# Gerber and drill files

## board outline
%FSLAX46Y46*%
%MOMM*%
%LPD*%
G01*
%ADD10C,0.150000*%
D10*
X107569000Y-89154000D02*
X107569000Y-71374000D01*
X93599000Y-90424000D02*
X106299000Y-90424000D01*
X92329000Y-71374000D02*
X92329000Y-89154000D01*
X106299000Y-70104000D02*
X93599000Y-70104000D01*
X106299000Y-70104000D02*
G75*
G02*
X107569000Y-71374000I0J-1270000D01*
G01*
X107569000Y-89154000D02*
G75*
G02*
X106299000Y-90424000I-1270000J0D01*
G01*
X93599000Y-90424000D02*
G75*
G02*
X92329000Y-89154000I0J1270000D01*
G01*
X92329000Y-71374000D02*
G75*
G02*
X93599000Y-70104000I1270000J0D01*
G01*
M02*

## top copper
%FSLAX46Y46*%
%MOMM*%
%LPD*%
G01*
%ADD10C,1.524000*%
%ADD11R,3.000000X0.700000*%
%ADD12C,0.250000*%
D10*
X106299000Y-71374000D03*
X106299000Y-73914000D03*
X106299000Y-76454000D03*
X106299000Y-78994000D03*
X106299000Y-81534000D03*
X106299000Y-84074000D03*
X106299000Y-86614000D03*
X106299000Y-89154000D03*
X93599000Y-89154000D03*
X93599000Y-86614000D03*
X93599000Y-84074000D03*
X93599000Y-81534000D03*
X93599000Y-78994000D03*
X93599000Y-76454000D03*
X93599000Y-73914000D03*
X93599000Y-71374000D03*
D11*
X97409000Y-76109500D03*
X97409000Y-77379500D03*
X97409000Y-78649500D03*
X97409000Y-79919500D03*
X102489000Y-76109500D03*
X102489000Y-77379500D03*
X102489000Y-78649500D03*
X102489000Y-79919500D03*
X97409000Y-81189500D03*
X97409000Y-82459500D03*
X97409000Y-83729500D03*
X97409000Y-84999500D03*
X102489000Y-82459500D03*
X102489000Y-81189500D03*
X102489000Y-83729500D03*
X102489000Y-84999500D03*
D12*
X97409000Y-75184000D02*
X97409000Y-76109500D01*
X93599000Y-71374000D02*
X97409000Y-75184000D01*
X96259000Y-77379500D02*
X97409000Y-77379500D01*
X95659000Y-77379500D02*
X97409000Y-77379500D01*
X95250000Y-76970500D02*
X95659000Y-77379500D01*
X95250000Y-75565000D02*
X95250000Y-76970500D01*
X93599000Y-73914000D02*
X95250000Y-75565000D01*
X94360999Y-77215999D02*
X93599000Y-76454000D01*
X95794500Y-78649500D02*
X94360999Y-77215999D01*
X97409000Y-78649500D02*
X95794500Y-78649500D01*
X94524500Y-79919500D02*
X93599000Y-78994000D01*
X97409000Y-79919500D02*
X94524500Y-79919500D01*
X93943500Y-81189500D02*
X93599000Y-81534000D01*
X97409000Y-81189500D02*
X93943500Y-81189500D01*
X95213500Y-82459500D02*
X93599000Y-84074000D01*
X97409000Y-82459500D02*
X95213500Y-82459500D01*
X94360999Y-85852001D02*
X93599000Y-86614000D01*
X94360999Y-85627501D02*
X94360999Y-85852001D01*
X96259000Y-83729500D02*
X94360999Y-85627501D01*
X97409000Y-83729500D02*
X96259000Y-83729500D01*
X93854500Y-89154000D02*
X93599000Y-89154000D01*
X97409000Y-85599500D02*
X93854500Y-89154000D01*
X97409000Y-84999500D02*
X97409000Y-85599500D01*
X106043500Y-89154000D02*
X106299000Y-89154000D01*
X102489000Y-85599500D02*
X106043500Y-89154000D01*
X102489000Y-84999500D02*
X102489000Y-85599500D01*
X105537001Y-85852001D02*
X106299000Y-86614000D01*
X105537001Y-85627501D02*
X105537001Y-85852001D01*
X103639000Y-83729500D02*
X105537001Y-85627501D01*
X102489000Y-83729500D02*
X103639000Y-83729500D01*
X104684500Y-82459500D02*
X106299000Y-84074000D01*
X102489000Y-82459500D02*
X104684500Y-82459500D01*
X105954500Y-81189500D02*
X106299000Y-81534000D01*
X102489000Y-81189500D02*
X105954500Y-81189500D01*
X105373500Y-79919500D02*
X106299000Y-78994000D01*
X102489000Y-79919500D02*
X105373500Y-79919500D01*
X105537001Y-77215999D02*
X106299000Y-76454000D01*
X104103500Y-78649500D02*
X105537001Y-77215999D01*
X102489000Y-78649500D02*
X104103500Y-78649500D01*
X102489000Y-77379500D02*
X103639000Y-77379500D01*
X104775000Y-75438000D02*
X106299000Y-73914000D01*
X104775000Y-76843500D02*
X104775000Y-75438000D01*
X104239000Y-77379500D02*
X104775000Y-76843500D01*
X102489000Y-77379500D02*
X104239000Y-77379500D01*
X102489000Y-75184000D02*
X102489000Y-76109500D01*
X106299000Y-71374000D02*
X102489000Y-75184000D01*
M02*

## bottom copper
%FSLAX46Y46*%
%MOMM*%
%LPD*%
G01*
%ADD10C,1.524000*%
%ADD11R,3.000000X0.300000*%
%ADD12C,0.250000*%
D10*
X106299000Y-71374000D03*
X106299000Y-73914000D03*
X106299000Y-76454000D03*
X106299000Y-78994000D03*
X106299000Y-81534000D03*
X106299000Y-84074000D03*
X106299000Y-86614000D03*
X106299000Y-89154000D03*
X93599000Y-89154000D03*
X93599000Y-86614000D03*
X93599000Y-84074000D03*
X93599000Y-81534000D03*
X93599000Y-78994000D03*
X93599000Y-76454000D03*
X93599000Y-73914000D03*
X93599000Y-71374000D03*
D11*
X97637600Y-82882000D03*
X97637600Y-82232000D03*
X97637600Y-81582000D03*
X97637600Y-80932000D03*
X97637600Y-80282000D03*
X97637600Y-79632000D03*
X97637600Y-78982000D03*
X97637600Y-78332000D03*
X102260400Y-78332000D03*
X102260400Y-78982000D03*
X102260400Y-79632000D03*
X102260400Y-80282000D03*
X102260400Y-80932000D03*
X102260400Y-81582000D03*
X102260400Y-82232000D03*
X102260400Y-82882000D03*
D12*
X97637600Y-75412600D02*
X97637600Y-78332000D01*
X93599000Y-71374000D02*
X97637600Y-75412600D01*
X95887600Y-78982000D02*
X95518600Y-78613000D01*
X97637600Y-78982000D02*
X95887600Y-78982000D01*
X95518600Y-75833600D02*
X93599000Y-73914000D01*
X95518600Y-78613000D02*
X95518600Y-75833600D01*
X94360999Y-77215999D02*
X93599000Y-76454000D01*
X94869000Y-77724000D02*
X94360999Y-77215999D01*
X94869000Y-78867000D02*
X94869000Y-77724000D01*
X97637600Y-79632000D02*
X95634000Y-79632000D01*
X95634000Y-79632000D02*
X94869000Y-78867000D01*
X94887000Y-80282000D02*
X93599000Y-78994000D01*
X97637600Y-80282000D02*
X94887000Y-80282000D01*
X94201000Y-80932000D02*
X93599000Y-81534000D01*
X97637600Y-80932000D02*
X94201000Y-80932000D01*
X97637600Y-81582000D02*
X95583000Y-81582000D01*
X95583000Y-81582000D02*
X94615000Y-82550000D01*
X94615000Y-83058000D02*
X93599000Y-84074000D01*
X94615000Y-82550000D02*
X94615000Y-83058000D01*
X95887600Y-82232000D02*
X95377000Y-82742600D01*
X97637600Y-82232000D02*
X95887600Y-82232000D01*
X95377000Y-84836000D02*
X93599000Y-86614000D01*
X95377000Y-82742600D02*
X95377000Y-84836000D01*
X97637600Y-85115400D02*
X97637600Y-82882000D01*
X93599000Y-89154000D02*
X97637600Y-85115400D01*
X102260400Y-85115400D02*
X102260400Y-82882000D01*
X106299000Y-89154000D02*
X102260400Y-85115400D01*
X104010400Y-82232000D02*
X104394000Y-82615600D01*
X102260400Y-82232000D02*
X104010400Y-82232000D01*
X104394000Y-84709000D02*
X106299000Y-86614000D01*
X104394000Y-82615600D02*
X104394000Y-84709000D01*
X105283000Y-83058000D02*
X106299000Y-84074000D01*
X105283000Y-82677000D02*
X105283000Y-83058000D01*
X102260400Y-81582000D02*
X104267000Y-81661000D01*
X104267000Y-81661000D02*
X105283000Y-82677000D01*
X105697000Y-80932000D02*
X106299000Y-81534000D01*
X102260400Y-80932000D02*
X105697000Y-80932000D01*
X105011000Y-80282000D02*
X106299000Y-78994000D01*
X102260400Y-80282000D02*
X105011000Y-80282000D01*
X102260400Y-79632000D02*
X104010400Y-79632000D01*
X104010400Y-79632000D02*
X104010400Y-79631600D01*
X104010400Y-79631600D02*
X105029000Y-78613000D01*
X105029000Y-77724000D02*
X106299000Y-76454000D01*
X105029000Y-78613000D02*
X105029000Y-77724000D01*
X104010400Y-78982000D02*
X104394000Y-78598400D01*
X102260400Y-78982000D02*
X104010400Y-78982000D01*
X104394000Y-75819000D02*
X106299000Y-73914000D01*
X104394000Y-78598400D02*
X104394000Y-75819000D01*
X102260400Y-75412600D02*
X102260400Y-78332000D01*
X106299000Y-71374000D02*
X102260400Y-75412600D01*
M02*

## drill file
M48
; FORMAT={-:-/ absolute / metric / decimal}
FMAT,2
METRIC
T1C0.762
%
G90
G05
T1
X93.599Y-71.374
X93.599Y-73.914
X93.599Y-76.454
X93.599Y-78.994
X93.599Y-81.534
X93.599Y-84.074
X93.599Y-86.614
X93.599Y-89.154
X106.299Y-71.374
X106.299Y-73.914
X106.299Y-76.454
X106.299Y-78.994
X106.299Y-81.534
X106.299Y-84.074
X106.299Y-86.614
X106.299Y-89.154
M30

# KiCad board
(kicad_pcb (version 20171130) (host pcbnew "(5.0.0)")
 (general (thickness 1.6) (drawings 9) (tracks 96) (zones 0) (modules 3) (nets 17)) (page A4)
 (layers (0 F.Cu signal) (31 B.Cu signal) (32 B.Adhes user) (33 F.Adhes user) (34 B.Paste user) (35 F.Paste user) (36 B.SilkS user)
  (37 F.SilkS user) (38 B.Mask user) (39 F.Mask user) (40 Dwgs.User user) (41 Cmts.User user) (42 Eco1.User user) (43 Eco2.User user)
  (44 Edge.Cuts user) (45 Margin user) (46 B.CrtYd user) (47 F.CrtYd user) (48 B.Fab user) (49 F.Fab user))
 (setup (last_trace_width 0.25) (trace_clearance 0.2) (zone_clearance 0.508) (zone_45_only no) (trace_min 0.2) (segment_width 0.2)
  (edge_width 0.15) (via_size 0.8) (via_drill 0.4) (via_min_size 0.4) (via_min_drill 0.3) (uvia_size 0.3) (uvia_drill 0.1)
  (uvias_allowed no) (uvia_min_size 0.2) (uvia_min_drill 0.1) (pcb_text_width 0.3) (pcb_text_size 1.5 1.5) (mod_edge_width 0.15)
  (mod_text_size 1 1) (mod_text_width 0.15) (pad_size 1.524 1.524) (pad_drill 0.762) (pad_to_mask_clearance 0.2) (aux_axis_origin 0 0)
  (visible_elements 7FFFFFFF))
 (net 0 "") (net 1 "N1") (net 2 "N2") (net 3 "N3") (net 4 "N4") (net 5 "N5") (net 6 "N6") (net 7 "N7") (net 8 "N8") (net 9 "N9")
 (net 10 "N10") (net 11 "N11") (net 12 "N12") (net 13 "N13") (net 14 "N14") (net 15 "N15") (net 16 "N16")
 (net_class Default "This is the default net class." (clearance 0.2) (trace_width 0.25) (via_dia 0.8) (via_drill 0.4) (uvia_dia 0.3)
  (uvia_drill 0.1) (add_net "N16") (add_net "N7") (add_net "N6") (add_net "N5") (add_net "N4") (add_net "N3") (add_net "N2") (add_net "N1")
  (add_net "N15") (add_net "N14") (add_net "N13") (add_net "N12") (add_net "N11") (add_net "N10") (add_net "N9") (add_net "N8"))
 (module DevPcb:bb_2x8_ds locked (layer F.Cu) (at 93.599 71.374)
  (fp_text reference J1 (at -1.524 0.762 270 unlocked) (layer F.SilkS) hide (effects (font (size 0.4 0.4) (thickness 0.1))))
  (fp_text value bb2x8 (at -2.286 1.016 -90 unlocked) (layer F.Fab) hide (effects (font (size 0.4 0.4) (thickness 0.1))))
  (pad 16 thru_hole circle (at 12.7 0) (size 1.524 1.524) (drill 0.762) (layers *.Cu *.Mask) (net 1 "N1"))
  (pad 15 thru_hole circle (at 12.7 2.54) (size 1.524 1.524) (drill 0.762) (layers *.Cu *.Mask) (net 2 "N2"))
  (pad 14 thru_hole circle (at 12.7 5.08) (size 1.524 1.524) (drill 0.762) (layers *.Cu *.Mask) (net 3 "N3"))
  (pad 13 thru_hole circle (at 12.7 7.62) (size 1.524 1.524) (drill 0.762) (layers *.Cu *.Mask) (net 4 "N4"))
  (pad 12 thru_hole circle (at 12.7 10.16) (size 1.524 1.524) (drill 0.762) (layers *.Cu *.Mask) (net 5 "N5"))
  (pad 11 thru_hole circle (at 12.7 12.7) (size 1.524 1.524) (drill 0.762) (layers *.Cu *.Mask) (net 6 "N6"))
  (pad 10 thru_hole circle (at 12.7 15.24) (size 1.524 1.524) (drill 0.762) (layers *.Cu *.Mask) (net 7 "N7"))
  (pad 9 thru_hole circle (at 12.7 17.78) (size 1.524 1.524) (drill 0.762) (layers *.Cu *.Mask) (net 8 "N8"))
  (pad 8 thru_hole circle (at 0 17.78) (size 1.524 1.524) (drill 0.762) (layers *.Cu *.Mask) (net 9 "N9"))
  (pad 7 thru_hole circle (at 0 15.24) (size 1.524 1.524) (drill 0.762) (layers *.Cu *.Mask) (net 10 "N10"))
  (pad 6 thru_hole circle (at 0 12.7) (size 1.524 1.524) (drill 0.762) (layers *.Cu *.Mask) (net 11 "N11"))
  (pad 5 thru_hole circle (at 0 10.16) (size 1.524 1.524) (drill 0.762) (layers *.Cu *.Mask) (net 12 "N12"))
  (pad 4 thru_hole circle (at 0 7.62) (size 1.524 1.524) (drill 0.762) (layers *.Cu *.Mask) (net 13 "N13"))
  (pad 3 thru_hole circle (at 0 5.08) (size 1.524 1.524) (drill 0.762) (layers *.Cu *.Mask) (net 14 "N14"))
  (pad 2 thru_hole circle (at 0 2.54) (size 1.524 1.524) (drill 0.762) (layers *.Cu *.Mask) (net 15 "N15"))
  (pad 1 thru_hole circle (at 0 0) (size 1.524 1.524) (drill 0.762) (layers *.Cu *.Mask) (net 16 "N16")))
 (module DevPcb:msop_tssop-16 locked (layer B.Cu) (at 99.9744 77.062 180)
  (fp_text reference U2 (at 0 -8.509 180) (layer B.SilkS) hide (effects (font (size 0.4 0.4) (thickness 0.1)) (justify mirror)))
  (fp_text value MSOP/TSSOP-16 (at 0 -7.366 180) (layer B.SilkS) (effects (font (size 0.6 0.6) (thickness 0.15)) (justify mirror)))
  (pad 9 smd rect (at 2.3368 -5.82 180) (size 3 0.3) (layers B.Cu B.Paste B.Mask) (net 9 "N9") (solder_mask_margin 0.1))
  (pad 10 smd rect (at 2.3368 -5.17 180) (size 3 0.3) (layers B.Cu B.Paste B.Mask) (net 10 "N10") (solder_mask_margin 0.1))
  (pad 11 smd rect (at 2.3368 -4.52 180) (size 3 0.3) (layers B.Cu B.Paste B.Mask) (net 11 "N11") (solder_mask_margin 0.1))
  (pad 12 smd rect (at 2.3368 -3.87 180) (size 3 0.3) (layers B.Cu B.Paste B.Mask) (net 12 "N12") (solder_mask_margin 0.1))
  (pad 13 smd rect (at 2.3368 -3.22 180) (size 3 0.3) (layers B.Cu B.Paste B.Mask) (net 13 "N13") (solder_mask_margin 0.1))
  (pad 14 smd rect (at 2.3368 -2.57 180) (size 3 0.3) (layers B.Cu B.Paste B.Mask) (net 14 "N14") (solder_mask_margin 0.1))
  (pad 15 smd rect (at 2.3368 -1.92 180) (size 3 0.3) (layers B.Cu B.Paste B.Mask) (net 15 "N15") (solder_mask_margin 0.1))
  (pad 16 smd rect (at 2.3368 -1.27) (size 3 0.3) (layers B.Cu B.Paste B.Mask) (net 16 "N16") (solder_mask_margin 0.1))
  (pad 1 smd rect (at -2.286 -1.27 180) (size 3 0.3) (layers B.Cu B.Paste B.Mask) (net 1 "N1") (solder_mask_margin 0.1))
  (pad 2 smd rect (at -2.286 -1.92 180) (size 3 0.3) (layers B.Cu B.Paste B.Mask) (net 2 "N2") (solder_mask_margin 0.1))
  (pad 3 smd rect (at -2.286 -2.57 180) (size 3 0.3) (layers B.Cu B.Paste B.Mask) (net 3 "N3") (solder_mask_margin 0.1))
  (pad 4 smd rect (at -2.286 -3.22 180) (size 3 0.3) (layers B.Cu B.Paste B.Mask) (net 4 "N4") (solder_mask_margin 0.1))
  (pad 5 smd rect (at -2.286 -3.87 180) (size 3 0.3) (layers B.Cu B.Paste B.Mask) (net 5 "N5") (solder_mask_margin 0.1))
  (pad 6 smd rect (at -2.286 -4.52 180) (size 3 0.3) (layers B.Cu B.Paste B.Mask) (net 6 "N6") (solder_mask_margin 0.1))
  (pad 7 smd rect (at -2.286 -5.17 180) (size 3 0.3) (layers B.Cu B.Paste B.Mask) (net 7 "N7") (solder_mask_margin 0.1))
  (pad 8 smd rect (at -2.286 -5.82 180) (size 3 0.3) (layers B.Cu B.Paste B.Mask) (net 8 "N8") (solder_mask_margin 0.1)))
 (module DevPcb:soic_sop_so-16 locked (layer F.Cu) (at 99.949 74.8395)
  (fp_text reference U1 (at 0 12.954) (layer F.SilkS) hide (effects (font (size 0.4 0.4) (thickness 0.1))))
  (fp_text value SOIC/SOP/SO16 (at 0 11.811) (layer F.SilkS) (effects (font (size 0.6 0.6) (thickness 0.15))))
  (pad 1 smd rect (at -2.54 1.27 90) (size 0.7 3) (layers F.Cu F.Paste F.Mask) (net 16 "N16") (solder_mask_margin 0.1))
  (pad 2 smd rect (at -2.54 2.54 90) (size 0.7 3) (layers F.Cu F.Paste F.Mask) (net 15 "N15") (solder_mask_margin 0.1))
  (pad 3 smd rect (at -2.54 3.81 90) (size 0.7 3) (layers F.Cu F.Paste F.Mask) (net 14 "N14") (solder_mask_margin 0.1))
  (pad 4 smd rect (at -2.54 5.08 90) (size 0.7 3) (layers F.Cu F.Paste F.Mask) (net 13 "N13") (solder_mask_margin 0.1))
  (pad 16 smd rect (at 2.54 1.27 90) (size 0.7 3) (layers F.Cu F.Paste F.Mask) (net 1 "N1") (solder_mask_margin 0.1))
  (pad 15 smd rect (at 2.54 2.54 90) (size 0.7 3) (layers F.Cu F.Paste F.Mask) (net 2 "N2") (solder_mask_margin 0.1))
  (pad 14 smd rect (at 2.54 3.81 90) (size 0.7 3) (layers F.Cu F.Paste F.Mask) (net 3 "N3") (solder_mask_margin 0.1))
  (pad 13 smd rect (at 2.54 5.08 90) (size 0.7 3) (layers F.Cu F.Paste F.Mask) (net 4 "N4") (solder_mask_margin 0.1))
  (pad 5 smd rect (at -2.54 6.35 90) (size 0.7 3) (layers F.Cu F.Paste F.Mask) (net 12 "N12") (solder_mask_margin 0.1))
  (pad 6 smd rect (at -2.54 7.62 90) (size 0.7 3) (layers F.Cu F.Paste F.Mask) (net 11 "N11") (solder_mask_margin 0.1))
  (pad 7 smd rect (at -2.54 8.89 90) (size 0.7 3) (layers F.Cu F.Paste F.Mask) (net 10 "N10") (solder_mask_margin 0.1))
  (pad 8 smd rect (at -2.54 10.16 90) (size 0.7 3) (layers F.Cu F.Paste F.Mask) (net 9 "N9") (solder_mask_margin 0.1))
  (pad 11 smd rect (at 2.54 7.62 90) (size 0.7 3) (layers F.Cu F.Paste F.Mask) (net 6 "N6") (solder_mask_margin 0.1))
  (pad 12 smd rect (at 2.54 6.35 90) (size 0.7 3) (layers F.Cu F.Paste F.Mask) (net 5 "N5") (solder_mask_margin 0.1))
  (pad 10 smd rect (at 2.54 8.89 90) (size 0.7 3) (layers F.Cu F.Paste F.Mask) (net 7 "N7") (solder_mask_margin 0.1))
  (pad 9 smd rect (at 2.54 10.16 90) (size 0.7 3) (layers F.Cu F.Paste F.Mask) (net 8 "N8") (solder_mask_margin 0.1)))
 (gr_line (start 107.569 89.154) (end 107.569 71.374) (layer Edge.Cuts) (width 0.15))
 (gr_line (start 93.599 90.424) (end 106.299 90.424) (layer Edge.Cuts) (width 0.15))
 (gr_line (start 92.329 71.374) (end 92.329 89.154) (layer Edge.Cuts) (width 0.15))
 (gr_line (start 106.299 70.104) (end 93.599 70.104) (layer Edge.Cuts) (width 0.15))
 (gr_arc (start 106.299 71.374) (end 107.569 71.374) (angle -90) (layer Edge.Cuts) (width 0.15))
 (gr_arc (start 106.299 89.154) (end 106.299 90.424) (angle -90) (layer Edge.Cuts) (width 0.15))
 (gr_arc (start 93.599 89.154) (end 92.329 89.154) (angle -90) (layer Edge.Cuts) (width 0.15))
 (gr_arc (start 93.599 71.374) (end 93.599 70.104) (angle -90) (layer Edge.Cuts) (width 0.15))
 (segment (start 97.409 75.184) (end 97.409 76.1095) (width 0.25) (layer F.Cu) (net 16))
 (segment (start 93.599 71.374) (end 97.409 75.184) (width 0.25) (layer F.Cu) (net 16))
 (segment (start 97.6376 75.4126) (end 97.6376 78.332) (width 0.25) (layer B.Cu) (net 16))
 (segment (start 93.599 71.374) (end 97.6376 75.4126) (width 0.25) (layer B.Cu) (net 16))
 (segment (start 96.259 77.3795) (end 97.409 77.3795) (width 0.25) (layer F.Cu) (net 15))
 (segment (start 95.659 77.3795) (end 97.409 77.3795) (width 0.25) (layer F.Cu) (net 15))
 (segment (start 95.25 76.9705) (end 95.659 77.3795) (width 0.25) (layer F.Cu) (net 15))
 (segment (start 95.25 75.565) (end 95.25 76.9705) (width 0.25) (layer F.Cu) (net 15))
 (segment (start 93.599 73.914) (end 95.25 75.565) (width 0.25) (layer F.Cu) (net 15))
 (segment (start 95.8876 78.982) (end 95.5186 78.613) (width 0.25) (layer B.Cu) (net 15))
 (segment (start 97.6376 78.982) (end 95.8876 78.982) (width 0.25) (layer B.Cu) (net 15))
 (segment (start 95.5186 75.8336) (end 93.599 73.914) (width 0.25) (layer B.Cu) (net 15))
 (segment (start 95.5186 78.613) (end 95.5186 75.8336) (width 0.25) (layer B.Cu) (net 15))
 (segment (start 94.360999 77.215999) (end 93.599 76.454) (width 0.25) (layer F.Cu) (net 14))
 (segment (start 95.7945 78.6495) (end 94.360999 77.215999) (width 0.25) (layer F.Cu) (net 14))
 (segment (start 97.409 78.6495) (end 95.7945 78.6495) (width 0.25) (layer F.Cu) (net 14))
 (segment (start 94.360999 77.215999) (end 93.599 76.454) (width 0.25) (layer B.Cu) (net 14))
 (segment (start 94.869 77.724) (end 94.360999 77.215999) (width 0.25) (layer B.Cu) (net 14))
 (segment (start 94.869 78.867) (end 94.869 77.724) (width 0.25) (layer B.Cu) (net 14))
 (segment (start 97.6376 79.632) (end 95.634 79.632) (width 0.25) (layer B.Cu) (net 14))
 (segment (start 95.634 79.632) (end 94.869 78.867) (width 0.25) (layer B.Cu) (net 14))
 (segment (start 94.5245 79.9195) (end 93.599 78.994) (width 0.25) (layer F.Cu) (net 13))
 (segment (start 97.409 79.9195) (end 94.5245 79.9195) (width 0.25) (layer F.Cu) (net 13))
 (segment (start 94.887 80.282) (end 93.599 78.994) (width 0.25) (layer B.Cu) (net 13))
 (segment (start 97.6376 80.282) (end 94.887 80.282) (width 0.25) (layer B.Cu) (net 13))
 (segment (start 93.9435 81.1895) (end 93.599 81.534) (width 0.25) (layer F.Cu) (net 12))
 (segment (start 97.409 81.1895) (end 93.9435 81.1895) (width 0.25) (layer F.Cu) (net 12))
 (segment (start 94.201 80.932) (end 93.599 81.534) (width 0.25) (layer B.Cu) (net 12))
 (segment (start 97.6376 80.932) (end 94.201 80.932) (width 0.25) (layer B.Cu) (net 12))
 (segment (start 95.2135 82.4595) (end 93.599 84.074) (width 0.25) (layer F.Cu) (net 11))
 (segment (start 97.409 82.4595) (end 95.2135 82.4595) (width 0.25) (layer F.Cu) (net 11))
 (segment (start 97.6376 81.582) (end 95.583 81.582) (width 0.25) (layer B.Cu) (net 11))
 (segment (start 95.583 81.582) (end 94.615 82.55) (width 0.25) (layer B.Cu) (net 11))
 (segment (start 94.615 83.058) (end 93.599 84.074) (width 0.25) (layer B.Cu) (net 11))
 (segment (start 94.615 82.55) (end 94.615 83.058) (width 0.25) (layer B.Cu) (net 11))
 (segment (start 94.360999 85.852001) (end 93.599 86.614) (width 0.25) (layer F.Cu) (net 10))
 (segment (start 94.360999 85.627501) (end 94.360999 85.852001) (width 0.25) (layer F.Cu) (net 10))
 (segment (start 96.259 83.7295) (end 94.360999 85.627501) (width 0.25) (layer F.Cu) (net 10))
 (segment (start 97.409 83.7295) (end 96.259 83.7295) (width 0.25) (layer F.Cu) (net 10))
 (segment (start 95.8876 82.232) (end 95.377 82.7426) (width 0.25) (layer B.Cu) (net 10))
 (segment (start 97.6376 82.232) (end 95.8876 82.232) (width 0.25) (layer B.Cu) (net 10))
 (segment (start 95.377 84.836) (end 93.599 86.614) (width 0.25) (layer B.Cu) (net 10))
 (segment (start 95.377 82.7426) (end 95.377 84.836) (width 0.25) (layer B.Cu) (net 10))
 (segment (start 93.8545 89.154) (end 93.599 89.154) (width 0.25) (layer F.Cu) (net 9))
 (segment (start 97.409 85.5995) (end 93.8545 89.154) (width 0.25) (layer F.Cu) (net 9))
 (segment (start 97.409 84.9995) (end 97.409 85.5995) (width 0.25) (layer F.Cu) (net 9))
 (segment (start 97.6376 85.1154) (end 97.6376 82.882) (width 0.25) (layer B.Cu) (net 9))
 (segment (start 93.599 89.154) (end 97.6376 85.1154) (width 0.25) (layer B.Cu) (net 9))
 (segment (start 106.0435 89.154) (end 106.299 89.154) (width 0.25) (layer F.Cu) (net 8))
 (segment (start 102.489 85.5995) (end 106.0435 89.154) (width 0.25) (layer F.Cu) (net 8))
 (segment (start 102.489 84.9995) (end 102.489 85.5995) (width 0.25) (layer F.Cu) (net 8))
 (segment (start 102.2604 85.1154) (end 102.2604 82.882) (width 0.25) (layer B.Cu) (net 8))
 (segment (start 106.299 89.154) (end 102.2604 85.1154) (width 0.25) (layer B.Cu) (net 8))
 (segment (start 105.537001 85.852001) (end 106.299 86.614) (width 0.25) (layer F.Cu) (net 7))
 (segment (start 105.537001 85.627501) (end 105.537001 85.852001) (width 0.25) (layer F.Cu) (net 7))
 (segment (start 103.639 83.7295) (end 105.537001 85.627501) (width 0.25) (layer F.Cu) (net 7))
 (segment (start 102.489 83.7295) (end 103.639 83.7295) (width 0.25) (layer F.Cu) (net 7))
 (segment (start 104.0104 82.232) (end 104.394 82.6156) (width 0.25) (layer B.Cu) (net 7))
 (segment (start 102.2604 82.232) (end 104.0104 82.232) (width 0.25) (layer B.Cu) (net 7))
 (segment (start 104.394 84.709) (end 106.299 86.614) (width 0.25) (layer B.Cu) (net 7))
 (segment (start 104.394 82.6156) (end 104.394 84.709) (width 0.25) (layer B.Cu) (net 7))
 (segment (start 104.6845 82.4595) (end 106.299 84.074) (width 0.25) (layer F.Cu) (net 6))
 (segment (start 102.489 82.4595) (end 104.6845 82.4595) (width 0.25) (layer F.Cu) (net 6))
 (segment (start 105.283 83.058) (end 106.299 84.074) (width 0.25) (layer B.Cu) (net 6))
 (segment (start 105.283 82.677) (end 105.283 83.058) (width 0.25) (layer B.Cu) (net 6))
 (segment (start 102.2604 81.582) (end 104.267 81.661) (width 0.25) (layer B.Cu) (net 6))
 (segment (start 104.267 81.661) (end 105.283 82.677) (width 0.25) (layer B.Cu) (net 6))
 (segment (start 105.9545 81.1895) (end 106.299 81.534) (width 0.25) (layer F.Cu) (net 5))
 (segment (start 102.489 81.1895) (end 105.9545 81.1895) (width 0.25) (layer F.Cu) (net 5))
 (segment (start 105.697 80.932) (end 106.299 81.534) (width 0.25) (layer B.Cu) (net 5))
 (segment (start 102.2604 80.932) (end 105.697 80.932) (width 0.25) (layer B.Cu) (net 5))
 (segment (start 105.3735 79.9195) (end 106.299 78.994) (width 0.25) (layer F.Cu) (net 4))
 (segment (start 102.489 79.9195) (end 105.3735 79.9195) (width 0.25) (layer F.Cu) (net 4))
 (segment (start 105.011 80.282) (end 106.299 78.994) (width 0.25) (layer B.Cu) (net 4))
 (segment (start 102.2604 80.282) (end 105.011 80.282) (width 0.25) (layer B.Cu) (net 4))
 (segment (start 105.537001 77.215999) (end 106.299 76.454) (width 0.25) (layer F.Cu) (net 3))
 (segment (start 104.1035 78.6495) (end 105.537001 77.215999) (width 0.25) (layer F.Cu) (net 3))
 (segment (start 102.489 78.6495) (end 104.1035 78.6495) (width 0.25) (layer F.Cu) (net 3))
 (segment (start 102.2604 79.632) (end 104.0104 79.632) (width 0.25) (layer B.Cu) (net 3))
 (segment (start 104.0104 79.632) (end 104.0104 79.6316) (width 0.25) (layer B.Cu) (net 3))
 (segment (start 104.0104 79.6316) (end 105.029 78.613) (width 0.25) (layer B.Cu) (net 3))
 (segment (start 105.029 77.724) (end 106.299 76.454) (width 0.25) (layer B.Cu) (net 3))
 (segment (start 105.029 78.613) (end 105.029 77.724) (width 0.25) (layer B.Cu) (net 3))
 (segment (start 102.489 77.3795) (end 103.639 77.3795) (width 0.25) (layer F.Cu) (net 2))
 (segment (start 104.775 75.438) (end 106.299 73.914) (width 0.25) (layer F.Cu) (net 2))
 (segment (start 104.775 76.8435) (end 104.775 75.438) (width 0.25) (layer F.Cu) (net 2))
 (segment (start 104.239 77.3795) (end 104.775 76.8435) (width 0.25) (layer F.Cu) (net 2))
 (segment (start 102.489 77.3795) (end 104.239 77.3795) (width 0.25) (layer F.Cu) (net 2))
 (segment (start 104.0104 78.982) (end 104.394 78.5984) (width 0.25) (layer B.Cu) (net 2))
 (segment (start 102.2604 78.982) (end 104.0104 78.982) (width 0.25) (layer B.Cu) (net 2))
 (segment (start 104.394 75.819) (end 106.299 73.914) (width 0.25) (layer B.Cu) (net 2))
 (segment (start 104.394 78.5984) (end 104.394 75.819) (width 0.25) (layer B.Cu) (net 2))
 (segment (start 102.489 75.184) (end 102.489 76.1095) (width 0.25) (layer F.Cu) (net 1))
 (segment (start 106.299 71.374) (end 102.489 75.184) (width 0.25) (layer F.Cu) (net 1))
 (segment (start 102.2604 75.4126) (end 102.2604 78.332) (width 0.25) (layer B.Cu) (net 1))
 (segment (start 106.299 71.374) (end 102.2604 75.4126) (width 0.25) (layer B.Cu) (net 1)))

